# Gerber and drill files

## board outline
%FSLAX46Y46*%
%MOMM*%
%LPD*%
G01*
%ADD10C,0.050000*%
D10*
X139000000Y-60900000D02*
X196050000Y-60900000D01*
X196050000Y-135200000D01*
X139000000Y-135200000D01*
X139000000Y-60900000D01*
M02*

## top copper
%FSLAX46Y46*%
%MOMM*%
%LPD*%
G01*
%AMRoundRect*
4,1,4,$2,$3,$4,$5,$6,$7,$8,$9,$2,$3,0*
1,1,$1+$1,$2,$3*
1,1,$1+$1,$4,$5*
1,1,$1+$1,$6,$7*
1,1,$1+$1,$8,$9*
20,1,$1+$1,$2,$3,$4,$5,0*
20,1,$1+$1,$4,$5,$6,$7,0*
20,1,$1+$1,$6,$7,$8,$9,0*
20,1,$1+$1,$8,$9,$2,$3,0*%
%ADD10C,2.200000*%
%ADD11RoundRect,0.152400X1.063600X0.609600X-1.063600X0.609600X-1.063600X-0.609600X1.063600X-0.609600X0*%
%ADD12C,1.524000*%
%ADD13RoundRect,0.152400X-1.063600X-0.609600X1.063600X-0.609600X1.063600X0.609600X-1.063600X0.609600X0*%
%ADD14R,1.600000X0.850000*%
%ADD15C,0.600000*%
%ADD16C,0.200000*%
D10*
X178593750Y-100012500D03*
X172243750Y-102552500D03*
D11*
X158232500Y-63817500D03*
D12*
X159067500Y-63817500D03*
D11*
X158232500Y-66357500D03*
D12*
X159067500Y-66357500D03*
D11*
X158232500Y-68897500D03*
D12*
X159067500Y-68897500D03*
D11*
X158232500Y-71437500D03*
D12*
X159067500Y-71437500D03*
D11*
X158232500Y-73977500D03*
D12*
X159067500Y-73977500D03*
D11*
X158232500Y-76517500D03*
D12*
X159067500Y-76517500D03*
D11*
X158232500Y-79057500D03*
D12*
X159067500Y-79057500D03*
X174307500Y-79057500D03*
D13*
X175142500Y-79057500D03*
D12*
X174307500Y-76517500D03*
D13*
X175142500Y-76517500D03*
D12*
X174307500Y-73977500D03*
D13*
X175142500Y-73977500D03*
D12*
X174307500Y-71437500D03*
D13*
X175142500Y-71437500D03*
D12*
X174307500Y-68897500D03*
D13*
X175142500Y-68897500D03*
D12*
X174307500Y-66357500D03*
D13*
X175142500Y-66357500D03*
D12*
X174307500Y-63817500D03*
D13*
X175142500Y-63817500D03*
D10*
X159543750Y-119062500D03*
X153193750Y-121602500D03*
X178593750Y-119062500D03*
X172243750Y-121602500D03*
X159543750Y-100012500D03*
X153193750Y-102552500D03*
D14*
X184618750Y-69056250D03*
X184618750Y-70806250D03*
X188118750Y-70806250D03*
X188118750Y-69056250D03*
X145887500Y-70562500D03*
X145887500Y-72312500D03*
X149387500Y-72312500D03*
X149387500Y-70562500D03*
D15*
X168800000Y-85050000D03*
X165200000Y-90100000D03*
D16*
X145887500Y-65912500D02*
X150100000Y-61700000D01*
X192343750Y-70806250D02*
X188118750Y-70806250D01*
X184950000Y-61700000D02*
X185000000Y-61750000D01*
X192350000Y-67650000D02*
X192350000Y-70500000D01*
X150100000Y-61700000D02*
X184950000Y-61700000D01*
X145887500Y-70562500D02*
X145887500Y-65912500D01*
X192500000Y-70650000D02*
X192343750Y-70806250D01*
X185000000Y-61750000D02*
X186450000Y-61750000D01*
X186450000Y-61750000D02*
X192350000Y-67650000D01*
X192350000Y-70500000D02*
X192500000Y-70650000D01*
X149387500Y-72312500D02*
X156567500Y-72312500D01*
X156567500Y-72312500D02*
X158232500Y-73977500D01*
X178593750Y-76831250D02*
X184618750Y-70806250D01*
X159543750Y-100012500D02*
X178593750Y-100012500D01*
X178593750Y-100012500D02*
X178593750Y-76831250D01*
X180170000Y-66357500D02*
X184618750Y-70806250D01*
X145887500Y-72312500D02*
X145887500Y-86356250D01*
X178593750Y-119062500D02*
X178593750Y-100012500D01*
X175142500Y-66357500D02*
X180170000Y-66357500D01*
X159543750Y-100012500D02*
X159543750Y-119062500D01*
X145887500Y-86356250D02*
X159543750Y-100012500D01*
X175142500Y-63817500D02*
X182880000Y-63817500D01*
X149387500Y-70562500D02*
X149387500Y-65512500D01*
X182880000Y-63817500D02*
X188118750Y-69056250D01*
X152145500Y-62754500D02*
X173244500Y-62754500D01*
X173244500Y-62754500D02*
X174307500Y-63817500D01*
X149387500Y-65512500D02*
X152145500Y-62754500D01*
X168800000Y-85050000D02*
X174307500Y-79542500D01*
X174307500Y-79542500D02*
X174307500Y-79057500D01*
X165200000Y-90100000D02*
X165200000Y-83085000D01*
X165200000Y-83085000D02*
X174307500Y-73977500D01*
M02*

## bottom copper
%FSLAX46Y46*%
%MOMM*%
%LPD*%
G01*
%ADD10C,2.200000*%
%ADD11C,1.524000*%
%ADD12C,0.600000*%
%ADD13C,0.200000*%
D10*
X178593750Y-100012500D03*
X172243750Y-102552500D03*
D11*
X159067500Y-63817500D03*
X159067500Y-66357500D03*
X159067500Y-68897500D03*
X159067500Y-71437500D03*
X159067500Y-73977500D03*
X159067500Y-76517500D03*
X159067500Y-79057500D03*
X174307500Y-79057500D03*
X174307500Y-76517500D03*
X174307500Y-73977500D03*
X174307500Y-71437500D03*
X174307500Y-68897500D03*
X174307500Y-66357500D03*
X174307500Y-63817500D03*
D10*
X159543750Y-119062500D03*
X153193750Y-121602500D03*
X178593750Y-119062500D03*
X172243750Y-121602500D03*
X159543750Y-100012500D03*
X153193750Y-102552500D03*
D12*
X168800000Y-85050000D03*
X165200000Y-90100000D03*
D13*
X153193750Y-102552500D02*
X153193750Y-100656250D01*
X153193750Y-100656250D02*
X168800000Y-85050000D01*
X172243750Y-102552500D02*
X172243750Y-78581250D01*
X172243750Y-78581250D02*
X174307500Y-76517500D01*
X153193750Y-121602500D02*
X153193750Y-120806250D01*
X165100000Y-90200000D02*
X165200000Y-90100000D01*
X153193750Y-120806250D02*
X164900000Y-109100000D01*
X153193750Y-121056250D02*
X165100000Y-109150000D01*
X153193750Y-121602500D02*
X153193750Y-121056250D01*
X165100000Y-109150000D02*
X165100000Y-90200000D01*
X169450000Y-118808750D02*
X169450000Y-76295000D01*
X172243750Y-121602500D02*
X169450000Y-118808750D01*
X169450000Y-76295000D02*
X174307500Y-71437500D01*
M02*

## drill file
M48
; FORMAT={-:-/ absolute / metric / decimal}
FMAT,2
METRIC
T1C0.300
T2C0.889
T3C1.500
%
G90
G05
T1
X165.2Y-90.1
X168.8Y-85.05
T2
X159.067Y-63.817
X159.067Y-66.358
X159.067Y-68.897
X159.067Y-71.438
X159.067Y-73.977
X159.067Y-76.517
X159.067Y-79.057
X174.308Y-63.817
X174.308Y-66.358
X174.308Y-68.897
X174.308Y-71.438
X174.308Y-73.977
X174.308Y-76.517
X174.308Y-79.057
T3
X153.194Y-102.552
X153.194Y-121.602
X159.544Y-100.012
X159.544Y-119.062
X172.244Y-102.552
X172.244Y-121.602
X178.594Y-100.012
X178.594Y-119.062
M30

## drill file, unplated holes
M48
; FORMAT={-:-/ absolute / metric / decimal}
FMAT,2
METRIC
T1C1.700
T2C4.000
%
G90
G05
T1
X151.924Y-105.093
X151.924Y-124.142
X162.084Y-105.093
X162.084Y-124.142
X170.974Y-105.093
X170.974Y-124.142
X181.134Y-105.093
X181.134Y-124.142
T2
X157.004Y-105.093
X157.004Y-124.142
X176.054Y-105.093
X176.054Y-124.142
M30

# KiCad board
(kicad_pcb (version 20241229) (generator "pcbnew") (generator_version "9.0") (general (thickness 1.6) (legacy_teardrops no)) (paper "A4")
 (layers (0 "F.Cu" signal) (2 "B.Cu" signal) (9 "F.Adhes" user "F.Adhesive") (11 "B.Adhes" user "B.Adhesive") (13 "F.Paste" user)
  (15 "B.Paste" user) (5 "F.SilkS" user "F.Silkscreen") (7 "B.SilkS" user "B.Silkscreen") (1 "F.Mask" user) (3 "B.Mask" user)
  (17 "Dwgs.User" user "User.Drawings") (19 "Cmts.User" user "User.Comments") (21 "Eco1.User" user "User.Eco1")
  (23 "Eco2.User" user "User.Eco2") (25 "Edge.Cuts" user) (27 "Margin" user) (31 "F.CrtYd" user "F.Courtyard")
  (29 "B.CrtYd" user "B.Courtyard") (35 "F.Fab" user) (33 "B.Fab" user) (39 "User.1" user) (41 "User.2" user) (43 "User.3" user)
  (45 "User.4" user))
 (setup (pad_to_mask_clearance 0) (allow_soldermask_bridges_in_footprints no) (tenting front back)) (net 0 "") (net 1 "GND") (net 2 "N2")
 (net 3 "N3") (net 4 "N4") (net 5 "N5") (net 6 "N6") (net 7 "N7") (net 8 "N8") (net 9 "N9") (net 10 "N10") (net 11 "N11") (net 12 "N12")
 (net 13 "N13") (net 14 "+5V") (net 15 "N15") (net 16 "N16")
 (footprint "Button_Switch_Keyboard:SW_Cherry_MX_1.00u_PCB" (layer "F.Cu") (at 178.59375 100.0125)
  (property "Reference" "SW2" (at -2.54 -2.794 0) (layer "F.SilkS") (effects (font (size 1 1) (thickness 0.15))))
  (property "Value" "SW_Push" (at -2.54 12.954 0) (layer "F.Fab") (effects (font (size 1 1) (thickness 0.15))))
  (pad "" np_thru_hole circle (at -7.62 5.08) (size 1.7 1.7) (drill 1.7) (layers "*.Cu" "*.Mask"))
  (pad "" np_thru_hole circle (at -2.54 5.08) (size 4 4) (drill 4) (layers "*.Cu" "*.Mask"))
  (pad "" np_thru_hole circle (at 2.54 5.08) (size 1.7 1.7) (drill 1.7) (layers "*.Cu" "*.Mask"))
  (pad "1" thru_hole circle (at 0 0) (size 2.2 2.2) (drill 1.5) (layers "*.Cu" "*.Mask") (remove_unused_layers no) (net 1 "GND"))
  (pad "2" thru_hole circle (at -6.35 2.54) (size 2.2 2.2) (drill 1.5) (layers "*.Cu" "*.Mask") (remove_unused_layers no) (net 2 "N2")))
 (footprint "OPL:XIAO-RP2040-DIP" (layer "F.Cu") (at 166.6875 71.4375)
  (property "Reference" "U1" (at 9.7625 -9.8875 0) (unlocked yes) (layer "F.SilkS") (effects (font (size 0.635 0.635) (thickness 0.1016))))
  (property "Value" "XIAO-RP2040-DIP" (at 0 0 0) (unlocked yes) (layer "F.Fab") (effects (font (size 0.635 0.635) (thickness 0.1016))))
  (pad "1" smd roundrect (at -8.455 -7.62 180) (size 2.432 1.524) (layers "F.Cu" "F.Mask") (roundrect_rratio 0.1) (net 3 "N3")
   (thermal_bridge_angle 45))
  (pad "1" thru_hole circle (at -7.62 -7.62 180) (size 1.524 1.524) (drill 0.889) (layers "*.Cu" "*.Mask") (remove_unused_layers no)
   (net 3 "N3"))
  (pad "2" smd roundrect (at -8.455 -5.08 180) (size 2.432 1.524) (layers "F.Cu" "F.Mask") (roundrect_rratio 0.1) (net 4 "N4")
   (thermal_bridge_angle 45))
  (pad "2" thru_hole circle (at -7.62 -5.08 180) (size 1.524 1.524) (drill 0.889) (layers "*.Cu" "*.Mask") (remove_unused_layers no)
   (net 4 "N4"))
  (pad "3" smd roundrect (at -8.455 -2.54 180) (size 2.432 1.524) (layers "F.Cu" "F.Mask") (roundrect_rratio 0.1) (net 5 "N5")
   (thermal_bridge_angle 45))
  (pad "3" thru_hole circle (at -7.62 -2.54 180) (size 1.524 1.524) (drill 0.889) (layers "*.Cu" "*.Mask") (remove_unused_layers no)
   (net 5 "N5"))
  (pad "4" smd roundrect (at -8.455 0 180) (size 2.432 1.524) (layers "F.Cu" "F.Mask") (roundrect_rratio 0.1) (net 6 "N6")
   (thermal_bridge_angle 45))
  (pad "4" thru_hole circle (at -7.62 0 180) (size 1.524 1.524) (drill 0.889) (layers "*.Cu" "*.Mask") (remove_unused_layers no)
   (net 6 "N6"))
  (pad "5" smd roundrect (at -8.455 2.54 180) (size 2.432 1.524) (layers "F.Cu" "F.Mask") (roundrect_rratio 0.1) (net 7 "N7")
   (thermal_bridge_angle 45))
  (pad "5" thru_hole circle (at -7.62 2.54 180) (size 1.524 1.524) (drill 0.889) (layers "*.Cu" "*.Mask") (remove_unused_layers no)
   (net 7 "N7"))
  (pad "6" smd roundrect (at -8.455 5.08 180) (size 2.432 1.524) (layers "F.Cu" "F.Mask") (roundrect_rratio 0.1) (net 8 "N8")
   (thermal_bridge_angle 45))
  (pad "6" thru_hole circle (at -7.62 5.08 180) (size 1.524 1.524) (drill 0.889) (layers "*.Cu" "*.Mask") (remove_unused_layers no)
   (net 8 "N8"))
  (pad "7" smd roundrect (at -8.455 7.62 180) (size 2.432 1.524) (layers "F.Cu" "F.Mask") (roundrect_rratio 0.1) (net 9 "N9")
   (thermal_bridge_angle 45))
  (pad "7" thru_hole circle (at -7.62 7.62 180) (size 1.524 1.524) (drill 0.889) (layers "*.Cu" "*.Mask") (remove_unused_layers no)
   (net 9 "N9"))
  (pad "8" thru_hole circle (at 7.62 7.62) (size 1.524 1.524) (drill 0.889) (layers "*.Cu" "*.Mask") (remove_unused_layers no)
   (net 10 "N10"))
  (pad "8" smd roundrect (at 8.455 7.62) (size 2.432 1.524) (layers "F.Cu" "F.Mask") (roundrect_rratio 0.1) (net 10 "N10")
   (thermal_bridge_angle 45))
  (pad "9" thru_hole circle (at 7.62 5.08) (size 1.524 1.524) (drill 0.889) (layers "*.Cu" "*.Mask") (remove_unused_layers no) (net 2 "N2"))
  (pad "9" smd roundrect (at 8.455 5.08) (size 2.432 1.524) (layers "F.Cu" "F.Mask") (roundrect_rratio 0.1) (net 2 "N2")
   (thermal_bridge_angle 45))
  (pad "10" thru_hole circle (at 7.62 2.54) (size 1.524 1.524) (drill 0.889) (layers "*.Cu" "*.Mask") (remove_unused_layers no)
   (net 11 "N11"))
  (pad "10" smd roundrect (at 8.455 2.54) (size 2.432 1.524) (layers "F.Cu" "F.Mask") (roundrect_rratio 0.1) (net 11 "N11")
   (thermal_bridge_angle 45))
  (pad "11" thru_hole circle (at 7.62 0) (size 1.524 1.524) (drill 0.889) (layers "*.Cu" "*.Mask") (remove_unused_layers no) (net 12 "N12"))
  (pad "11" smd roundrect (at 8.455 0) (size 2.432 1.524) (layers "F.Cu" "F.Mask") (roundrect_rratio 0.1) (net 12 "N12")
   (thermal_bridge_angle 45))
  (pad "12" thru_hole circle (at 7.62 -2.54) (size 1.524 1.524) (drill 0.889) (layers "*.Cu" "*.Mask") (remove_unused_layers no)
   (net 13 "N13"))
  (pad "12" smd roundrect (at 8.455 -2.54) (size 2.432 1.524) (layers "F.Cu" "F.Mask") (roundrect_rratio 0.1) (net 13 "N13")
   (thermal_bridge_angle 45))
  (pad "13" thru_hole circle (at 7.62 -5.08) (size 1.524 1.524) (drill 0.889) (layers "*.Cu" "*.Mask") (remove_unused_layers no)
   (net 1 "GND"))
  (pad "13" smd roundrect (at 8.455 -5.08) (size 2.432 1.524) (layers "F.Cu" "F.Mask") (roundrect_rratio 0.1) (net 1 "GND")
   (thermal_bridge_angle 45))
  (pad "14" thru_hole circle (at 7.62 -7.62) (size 1.524 1.524) (drill 0.889) (layers "*.Cu" "*.Mask") (remove_unused_layers no)
   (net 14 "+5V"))
  (pad "14" smd roundrect (at 8.455 -7.62) (size 2.432 1.524) (layers "F.Cu" "F.Mask") (roundrect_rratio 0.1) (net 14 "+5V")
   (thermal_bridge_angle 45)))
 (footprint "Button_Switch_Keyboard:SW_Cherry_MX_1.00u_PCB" (layer "F.Cu") (at 159.54375 119.0625)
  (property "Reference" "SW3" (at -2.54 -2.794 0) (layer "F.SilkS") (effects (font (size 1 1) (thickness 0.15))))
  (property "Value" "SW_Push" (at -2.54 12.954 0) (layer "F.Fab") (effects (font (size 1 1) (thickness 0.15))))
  (pad "" np_thru_hole circle (at -7.62 5.08) (size 1.7 1.7) (drill 1.7) (layers "*.Cu" "*.Mask"))
  (pad "" np_thru_hole circle (at -2.54 5.08) (size 4 4) (drill 4) (layers "*.Cu" "*.Mask"))
  (pad "" np_thru_hole circle (at 2.54 5.08) (size 1.7 1.7) (drill 1.7) (layers "*.Cu" "*.Mask"))
  (pad "1" thru_hole circle (at 0 0) (size 2.2 2.2) (drill 1.5) (layers "*.Cu" "*.Mask") (remove_unused_layers no) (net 1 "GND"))
  (pad "2" thru_hole circle (at -6.35 2.54) (size 2.2 2.2) (drill 1.5) (layers "*.Cu" "*.Mask") (remove_unused_layers no) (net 11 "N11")))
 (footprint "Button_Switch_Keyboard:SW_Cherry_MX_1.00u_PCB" (layer "F.Cu") (at 178.59375 119.0625)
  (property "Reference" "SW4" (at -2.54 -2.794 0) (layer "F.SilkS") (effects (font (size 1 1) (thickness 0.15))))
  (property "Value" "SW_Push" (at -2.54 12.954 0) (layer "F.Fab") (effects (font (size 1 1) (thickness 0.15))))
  (pad "" np_thru_hole circle (at -7.62 5.08) (size 1.7 1.7) (drill 1.7) (layers "*.Cu" "*.Mask"))
  (pad "" np_thru_hole circle (at -2.54 5.08) (size 4 4) (drill 4) (layers "*.Cu" "*.Mask"))
  (pad "" np_thru_hole circle (at 2.54 5.08) (size 1.7 1.7) (drill 1.7) (layers "*.Cu" "*.Mask"))
  (pad "1" thru_hole circle (at 0 0) (size 2.2 2.2) (drill 1.5) (layers "*.Cu" "*.Mask") (remove_unused_layers no) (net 1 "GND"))
  (pad "2" thru_hole circle (at -6.35 2.54) (size 2.2 2.2) (drill 1.5) (layers "*.Cu" "*.Mask") (remove_unused_layers no) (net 12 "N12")))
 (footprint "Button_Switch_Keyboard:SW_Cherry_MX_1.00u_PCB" (layer "F.Cu") (at 159.54375 100.0125)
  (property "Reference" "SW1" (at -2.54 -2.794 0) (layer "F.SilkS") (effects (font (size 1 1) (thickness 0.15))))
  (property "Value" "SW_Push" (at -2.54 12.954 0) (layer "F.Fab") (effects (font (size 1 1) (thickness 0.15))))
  (pad "" np_thru_hole circle (at -7.62 5.08) (size 1.7 1.7) (drill 1.7) (layers "*.Cu" "*.Mask"))
  (pad "" np_thru_hole circle (at -2.54 5.08) (size 4 4) (drill 4) (layers "*.Cu" "*.Mask"))
  (pad "" np_thru_hole circle (at 2.54 5.08) (size 1.7 1.7) (drill 1.7) (layers "*.Cu" "*.Mask"))
  (pad "1" thru_hole circle (at 0 0) (size 2.2 2.2) (drill 1.5) (layers "*.Cu" "*.Mask") (remove_unused_layers no) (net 1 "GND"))
  (pad "2" thru_hole circle (at -6.35 2.54) (size 2.2 2.2) (drill 1.5) (layers "*.Cu" "*.Mask") (remove_unused_layers no) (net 10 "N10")))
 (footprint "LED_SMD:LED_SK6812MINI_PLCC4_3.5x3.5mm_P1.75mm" (layer "F.Cu") (at 186.36875 69.93125)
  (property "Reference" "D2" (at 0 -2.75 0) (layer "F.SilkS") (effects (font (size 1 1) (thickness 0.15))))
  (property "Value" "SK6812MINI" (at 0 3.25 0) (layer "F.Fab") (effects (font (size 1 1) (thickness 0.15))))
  (pad "1" smd rect (at -1.75 -0.875) (size 1.6 0.85) (layers "F.Cu" "F.Mask" "F.Paste") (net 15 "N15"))
  (pad "2" smd rect (at -1.75 0.875) (size 1.6 0.85) (layers "F.Cu" "F.Mask" "F.Paste") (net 1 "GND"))
  (pad "3" smd rect (at 1.75 0.875) (size 1.6 0.85) (layers "F.Cu" "F.Mask" "F.Paste") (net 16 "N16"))
  (pad "4" smd rect (at 1.75 -0.875) (size 1.6 0.85) (layers "F.Cu" "F.Mask" "F.Paste") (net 14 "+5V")))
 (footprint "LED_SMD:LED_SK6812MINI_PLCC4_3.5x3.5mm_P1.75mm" (layer "F.Cu") (at 147.6375 71.4375)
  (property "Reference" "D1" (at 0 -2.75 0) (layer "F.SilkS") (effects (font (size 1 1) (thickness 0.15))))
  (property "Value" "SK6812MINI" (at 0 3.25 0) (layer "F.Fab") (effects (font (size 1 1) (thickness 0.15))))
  (pad "1" smd rect (at -1.75 -0.875) (size 1.6 0.85) (layers "F.Cu" "F.Mask" "F.Paste") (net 16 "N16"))
  (pad "2" smd rect (at -1.75 0.875) (size 1.6 0.85) (layers "F.Cu" "F.Mask" "F.Paste") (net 1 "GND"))
  (pad "3" smd rect (at 1.75 0.875) (size 1.6 0.85) (layers "F.Cu" "F.Mask" "F.Paste") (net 7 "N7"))
  (pad "4" smd rect (at 1.75 -0.875) (size 1.6 0.85) (layers "F.Cu" "F.Mask" "F.Paste") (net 14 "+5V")))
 (gr_rect (start 139 60.9) (end 196.05 135.2) (stroke (width 0.05) (type default)) (fill no) (layer "Edge.Cuts"))
 (segment (start 145.8875 65.9125) (end 150.1 61.7) (width 0.2) (layer "F.Cu") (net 16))
 (segment (start 192.34375 70.80625) (end 188.11875 70.80625) (width 0.2) (layer "F.Cu") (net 16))
 (segment (start 184.95 61.7) (end 185 61.75) (width 0.2) (layer "F.Cu") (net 16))
 (segment (start 192.35 67.65) (end 192.35 70.5) (width 0.2) (layer "F.Cu") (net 16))
 (segment (start 150.1 61.7) (end 184.95 61.7) (width 0.2) (layer "F.Cu") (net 16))
 (segment (start 145.8875 70.5625) (end 145.8875 65.9125) (width 0.2) (layer "F.Cu") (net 16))
 (segment (start 192.5 70.65) (end 192.34375 70.80625) (width 0.2) (layer "F.Cu") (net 16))
 (segment (start 185 61.75) (end 186.45 61.75) (width 0.2) (layer "F.Cu") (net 16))
 (segment (start 186.45 61.75) (end 192.35 67.65) (width 0.2) (layer "F.Cu") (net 16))
 (segment (start 192.35 70.5) (end 192.5 70.65) (width 0.2) (layer "F.Cu") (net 16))
 (segment (start 149.3875 72.3125) (end 156.5675 72.3125) (width 0.2) (layer "F.Cu") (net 7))
 (segment (start 156.5675 72.3125) (end 158.2325 73.9775) (width 0.2) (layer "F.Cu") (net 7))
 (segment (start 178.59375 76.83125) (end 184.61875 70.80625) (width 0.2) (layer "F.Cu") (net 1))
 (segment (start 159.54375 100.0125) (end 178.59375 100.0125) (width 0.2) (layer "F.Cu") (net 1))
 (segment (start 178.59375 100.0125) (end 178.59375 76.83125) (width 0.2) (layer "F.Cu") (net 1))
 (segment (start 180.17 66.3575) (end 184.61875 70.80625) (width 0.2) (layer "F.Cu") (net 1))
 (segment (start 145.8875 72.3125) (end 145.8875 86.35625) (width 0.2) (layer "F.Cu") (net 1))
 (segment (start 178.59375 119.0625) (end 178.59375 100.0125) (width 0.2) (layer "F.Cu") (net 1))
 (segment (start 175.1425 66.3575) (end 180.17 66.3575) (width 0.2) (layer "F.Cu") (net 1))
 (segment (start 159.54375 100.0125) (end 159.54375 119.0625) (width 0.2) (layer "F.Cu") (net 1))
 (segment (start 145.8875 86.35625) (end 159.54375 100.0125) (width 0.2) (layer "F.Cu") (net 1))
 (segment (start 175.1425 63.8175) (end 182.88 63.8175) (width 0.2) (layer "F.Cu") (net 14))
 (segment (start 149.3875 70.5625) (end 149.3875 65.5125) (width 0.2) (layer "F.Cu") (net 14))
 (segment (start 182.88 63.8175) (end 188.11875 69.05625) (width 0.2) (layer "F.Cu") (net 14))
 (segment (start 152.1455 62.7545) (end 173.2445 62.7545) (width 0.2) (layer "F.Cu") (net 14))
 (segment (start 173.2445 62.7545) (end 174.3075 63.8175) (width 0.2) (layer "F.Cu") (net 14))
 (segment (start 149.3875 65.5125) (end 152.1455 62.7545) (width 0.2) (layer "F.Cu") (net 14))
 (segment (start 168.8 85.05) (end 174.3075 79.5425) (width 0.2) (layer "F.Cu") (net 10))
 (segment (start 174.3075 79.5425) (end 174.3075 79.0575) (width 0.2) (layer "F.Cu") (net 10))
 (via (at 168.8 85.05) (size 0.6) (drill 0.3) (layers "F.Cu" "B.Cu") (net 10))
 (segment (start 153.19375 102.5525) (end 153.19375 100.65625) (width 0.2) (layer "B.Cu") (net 10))
 (segment (start 153.19375 100.65625) (end 168.8 85.05) (width 0.2) (layer "B.Cu") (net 10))
 (segment (start 172.24375 102.5525) (end 172.24375 78.58125) (width 0.2) (layer "B.Cu") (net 2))
 (segment (start 172.24375 78.58125) (end 174.3075 76.5175) (width 0.2) (layer "B.Cu") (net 2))
 (segment (start 165.2 90.1) (end 165.2 83.085) (width 0.2) (layer "F.Cu") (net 11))
 (segment (start 165.2 83.085) (end 174.3075 73.9775) (width 0.2) (layer "F.Cu") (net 11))
 (via (at 165.2 90.1) (size 0.6) (drill 0.3) (layers "F.Cu" "B.Cu") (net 11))
 (segment (start 153.19375 121.6025) (end 153.19375 120.80625) (width 0.2) (layer "B.Cu") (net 11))
 (segment (start 165.1 90.2) (end 165.2 90.1) (width 0.2) (layer "B.Cu") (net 11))
 (segment (start 153.19375 120.80625) (end 164.9 109.1) (width 0.2) (layer "B.Cu") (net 11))
 (segment (start 153.19375 121.05625) (end 165.1 109.15) (width 0.2) (layer "B.Cu") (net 11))
 (segment (start 153.19375 121.6025) (end 153.19375 121.05625) (width 0.2) (layer "B.Cu") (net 11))
 (segment (start 165.1 109.15) (end 165.1 90.2) (width 0.2) (layer "B.Cu") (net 11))
 (segment (start 169.45 118.80875) (end 169.45 76.295) (width 0.2) (layer "B.Cu") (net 12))
 (segment (start 172.24375 121.6025) (end 169.45 118.80875) (width 0.2) (layer "B.Cu") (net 12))
 (segment (start 169.45 76.295) (end 174.3075 71.4375) (width 0.2) (layer "B.Cu") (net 12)))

